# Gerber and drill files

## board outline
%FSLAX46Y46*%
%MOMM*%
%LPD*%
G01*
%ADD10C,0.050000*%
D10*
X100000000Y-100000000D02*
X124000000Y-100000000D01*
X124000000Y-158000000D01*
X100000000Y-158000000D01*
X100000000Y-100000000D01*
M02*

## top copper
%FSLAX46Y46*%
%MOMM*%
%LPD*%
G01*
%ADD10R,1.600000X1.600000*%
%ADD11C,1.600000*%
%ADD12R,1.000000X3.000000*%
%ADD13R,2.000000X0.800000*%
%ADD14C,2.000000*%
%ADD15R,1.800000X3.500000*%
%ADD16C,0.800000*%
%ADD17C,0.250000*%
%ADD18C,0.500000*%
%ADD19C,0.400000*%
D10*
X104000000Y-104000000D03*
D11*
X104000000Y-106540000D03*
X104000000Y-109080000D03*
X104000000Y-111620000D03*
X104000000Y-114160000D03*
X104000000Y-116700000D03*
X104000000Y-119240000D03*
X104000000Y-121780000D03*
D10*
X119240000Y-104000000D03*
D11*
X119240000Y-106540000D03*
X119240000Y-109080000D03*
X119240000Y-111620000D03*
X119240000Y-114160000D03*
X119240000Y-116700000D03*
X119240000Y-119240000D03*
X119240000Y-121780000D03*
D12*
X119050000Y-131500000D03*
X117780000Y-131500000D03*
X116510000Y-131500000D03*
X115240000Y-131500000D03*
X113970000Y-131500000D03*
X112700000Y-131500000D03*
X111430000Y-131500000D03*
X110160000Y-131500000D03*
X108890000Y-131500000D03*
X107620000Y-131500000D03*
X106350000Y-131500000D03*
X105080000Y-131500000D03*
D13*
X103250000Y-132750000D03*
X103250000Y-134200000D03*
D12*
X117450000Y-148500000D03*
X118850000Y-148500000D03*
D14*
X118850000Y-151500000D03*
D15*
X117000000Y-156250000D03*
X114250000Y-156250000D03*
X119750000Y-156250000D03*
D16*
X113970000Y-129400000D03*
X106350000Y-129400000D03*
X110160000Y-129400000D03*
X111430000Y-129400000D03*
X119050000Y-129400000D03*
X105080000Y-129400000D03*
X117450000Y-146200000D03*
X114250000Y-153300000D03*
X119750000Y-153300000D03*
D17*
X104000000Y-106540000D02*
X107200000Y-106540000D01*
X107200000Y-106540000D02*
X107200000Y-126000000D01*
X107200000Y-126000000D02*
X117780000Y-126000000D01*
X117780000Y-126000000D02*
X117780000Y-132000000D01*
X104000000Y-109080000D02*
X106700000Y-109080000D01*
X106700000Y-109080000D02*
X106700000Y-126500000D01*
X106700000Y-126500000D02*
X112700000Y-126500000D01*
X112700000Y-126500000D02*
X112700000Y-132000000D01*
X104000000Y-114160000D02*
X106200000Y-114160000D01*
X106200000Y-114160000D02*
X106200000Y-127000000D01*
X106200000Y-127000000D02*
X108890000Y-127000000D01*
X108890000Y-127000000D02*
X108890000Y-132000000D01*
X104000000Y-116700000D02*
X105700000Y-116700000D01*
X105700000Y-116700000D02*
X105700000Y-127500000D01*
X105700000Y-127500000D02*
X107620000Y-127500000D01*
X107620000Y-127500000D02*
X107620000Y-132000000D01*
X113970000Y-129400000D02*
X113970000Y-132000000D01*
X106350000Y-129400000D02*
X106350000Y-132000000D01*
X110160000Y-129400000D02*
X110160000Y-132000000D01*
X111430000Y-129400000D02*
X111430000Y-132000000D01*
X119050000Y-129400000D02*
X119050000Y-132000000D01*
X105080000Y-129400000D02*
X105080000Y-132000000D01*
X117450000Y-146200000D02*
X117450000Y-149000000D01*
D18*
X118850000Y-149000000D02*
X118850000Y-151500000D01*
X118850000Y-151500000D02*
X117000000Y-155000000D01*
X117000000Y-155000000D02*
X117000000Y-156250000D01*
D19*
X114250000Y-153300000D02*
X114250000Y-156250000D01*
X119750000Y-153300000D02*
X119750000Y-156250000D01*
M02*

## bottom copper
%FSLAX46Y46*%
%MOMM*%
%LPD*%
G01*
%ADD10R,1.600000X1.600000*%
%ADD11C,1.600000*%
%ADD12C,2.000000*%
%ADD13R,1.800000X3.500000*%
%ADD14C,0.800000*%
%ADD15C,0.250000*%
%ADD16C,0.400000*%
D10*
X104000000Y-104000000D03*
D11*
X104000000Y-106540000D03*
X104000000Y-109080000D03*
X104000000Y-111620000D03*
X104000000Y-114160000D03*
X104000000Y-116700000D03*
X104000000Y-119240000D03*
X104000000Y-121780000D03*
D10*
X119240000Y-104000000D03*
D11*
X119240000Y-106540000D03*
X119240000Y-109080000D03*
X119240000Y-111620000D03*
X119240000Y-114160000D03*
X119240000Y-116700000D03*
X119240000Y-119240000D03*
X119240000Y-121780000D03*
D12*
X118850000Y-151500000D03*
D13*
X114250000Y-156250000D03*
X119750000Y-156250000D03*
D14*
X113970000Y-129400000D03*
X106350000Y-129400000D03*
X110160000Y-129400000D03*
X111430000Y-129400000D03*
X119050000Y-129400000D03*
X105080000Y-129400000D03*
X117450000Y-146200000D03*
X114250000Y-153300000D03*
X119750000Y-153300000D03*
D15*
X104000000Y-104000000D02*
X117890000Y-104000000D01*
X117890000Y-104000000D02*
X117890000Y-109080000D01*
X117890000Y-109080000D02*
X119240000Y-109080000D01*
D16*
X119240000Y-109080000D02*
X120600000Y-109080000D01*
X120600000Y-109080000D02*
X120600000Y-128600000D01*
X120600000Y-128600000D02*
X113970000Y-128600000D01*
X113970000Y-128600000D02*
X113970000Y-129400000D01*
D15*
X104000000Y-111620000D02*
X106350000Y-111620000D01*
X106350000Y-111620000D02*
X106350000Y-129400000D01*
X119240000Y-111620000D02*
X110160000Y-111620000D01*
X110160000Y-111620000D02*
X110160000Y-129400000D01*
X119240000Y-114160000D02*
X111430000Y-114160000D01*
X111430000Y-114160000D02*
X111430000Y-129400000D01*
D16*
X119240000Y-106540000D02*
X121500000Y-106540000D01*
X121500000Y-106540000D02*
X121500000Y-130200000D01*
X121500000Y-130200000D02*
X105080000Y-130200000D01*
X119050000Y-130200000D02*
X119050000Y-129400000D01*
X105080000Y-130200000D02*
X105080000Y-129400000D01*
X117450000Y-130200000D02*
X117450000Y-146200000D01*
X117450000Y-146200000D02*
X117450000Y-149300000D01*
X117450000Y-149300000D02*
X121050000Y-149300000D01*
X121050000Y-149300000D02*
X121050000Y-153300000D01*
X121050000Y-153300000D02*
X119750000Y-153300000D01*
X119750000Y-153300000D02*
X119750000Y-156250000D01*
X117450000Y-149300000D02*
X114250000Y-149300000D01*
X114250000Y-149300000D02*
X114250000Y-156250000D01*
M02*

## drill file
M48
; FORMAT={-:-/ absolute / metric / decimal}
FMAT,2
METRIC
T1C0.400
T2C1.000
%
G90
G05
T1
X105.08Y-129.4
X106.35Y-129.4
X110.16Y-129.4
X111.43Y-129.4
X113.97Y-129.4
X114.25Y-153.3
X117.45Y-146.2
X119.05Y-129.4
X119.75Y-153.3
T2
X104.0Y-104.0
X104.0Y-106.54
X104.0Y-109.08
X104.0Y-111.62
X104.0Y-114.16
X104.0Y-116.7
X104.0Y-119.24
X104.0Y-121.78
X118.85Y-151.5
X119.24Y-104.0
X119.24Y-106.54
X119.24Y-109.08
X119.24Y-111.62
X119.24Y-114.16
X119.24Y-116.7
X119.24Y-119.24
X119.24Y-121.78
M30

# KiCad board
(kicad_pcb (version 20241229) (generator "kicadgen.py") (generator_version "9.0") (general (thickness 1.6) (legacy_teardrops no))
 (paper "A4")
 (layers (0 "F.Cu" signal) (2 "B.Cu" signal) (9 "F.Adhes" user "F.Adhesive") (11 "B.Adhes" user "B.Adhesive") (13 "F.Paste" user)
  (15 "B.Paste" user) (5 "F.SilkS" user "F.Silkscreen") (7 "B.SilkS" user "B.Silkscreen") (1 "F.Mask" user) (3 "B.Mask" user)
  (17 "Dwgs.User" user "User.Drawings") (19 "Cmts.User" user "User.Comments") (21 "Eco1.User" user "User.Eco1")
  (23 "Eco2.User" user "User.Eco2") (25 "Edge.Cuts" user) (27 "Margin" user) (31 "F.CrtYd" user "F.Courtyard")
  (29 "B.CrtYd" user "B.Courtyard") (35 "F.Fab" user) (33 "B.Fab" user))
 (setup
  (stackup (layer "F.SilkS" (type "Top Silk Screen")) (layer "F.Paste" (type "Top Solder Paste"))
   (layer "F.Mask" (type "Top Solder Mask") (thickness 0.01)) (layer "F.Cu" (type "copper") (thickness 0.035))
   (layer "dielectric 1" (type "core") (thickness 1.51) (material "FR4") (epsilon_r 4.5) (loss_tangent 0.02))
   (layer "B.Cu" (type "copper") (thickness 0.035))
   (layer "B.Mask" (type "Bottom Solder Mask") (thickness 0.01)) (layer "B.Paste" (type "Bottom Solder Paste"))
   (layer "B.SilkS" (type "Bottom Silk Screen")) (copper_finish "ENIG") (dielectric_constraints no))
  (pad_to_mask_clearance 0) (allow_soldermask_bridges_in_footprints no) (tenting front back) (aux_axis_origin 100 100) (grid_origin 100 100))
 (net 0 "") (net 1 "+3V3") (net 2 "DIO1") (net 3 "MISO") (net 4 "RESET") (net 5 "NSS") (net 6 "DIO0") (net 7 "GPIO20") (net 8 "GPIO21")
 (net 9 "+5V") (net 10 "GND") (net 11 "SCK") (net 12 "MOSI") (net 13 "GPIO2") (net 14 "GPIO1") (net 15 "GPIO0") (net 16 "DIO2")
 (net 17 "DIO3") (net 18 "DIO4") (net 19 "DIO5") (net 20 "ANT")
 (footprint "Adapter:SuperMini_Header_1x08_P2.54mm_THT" (layer "F.Cu") (at 104 104)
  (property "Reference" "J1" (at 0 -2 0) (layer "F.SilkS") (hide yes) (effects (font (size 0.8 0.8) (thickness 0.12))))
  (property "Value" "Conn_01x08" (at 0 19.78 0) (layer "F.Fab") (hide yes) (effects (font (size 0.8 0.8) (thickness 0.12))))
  (pad "1" thru_hole rect (at 0 0) (size 1.6 1.6) (drill 1) (layers "*.Cu" "*.Mask") (remove_unused_layers no) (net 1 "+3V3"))
  (pad "2" thru_hole circle (at 0 2.54) (size 1.6 1.6) (drill 1) (layers "*.Cu" "*.Mask") (remove_unused_layers no) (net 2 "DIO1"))
  (pad "3" thru_hole circle (at 0 5.08) (size 1.6 1.6) (drill 1) (layers "*.Cu" "*.Mask") (remove_unused_layers no) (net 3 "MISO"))
  (pad "4" thru_hole circle (at 0 7.62) (size 1.6 1.6) (drill 1) (layers "*.Cu" "*.Mask") (remove_unused_layers no) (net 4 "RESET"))
  (pad "5" thru_hole circle (at 0 10.16) (size 1.6 1.6) (drill 1) (layers "*.Cu" "*.Mask") (remove_unused_layers no) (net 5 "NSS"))
  (pad "6" thru_hole circle (at 0 12.7) (size 1.6 1.6) (drill 1) (layers "*.Cu" "*.Mask") (remove_unused_layers no) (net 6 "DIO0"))
  (pad "7" thru_hole circle (at 0 15.24) (size 1.6 1.6) (drill 1) (layers "*.Cu" "*.Mask") (remove_unused_layers no) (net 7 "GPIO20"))
  (pad "8" thru_hole circle (at 0 17.78) (size 1.6 1.6) (drill 1) (layers "*.Cu" "*.Mask") (remove_unused_layers no) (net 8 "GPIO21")))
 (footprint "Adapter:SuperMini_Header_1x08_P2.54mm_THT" (layer "F.Cu") (at 119.24 104)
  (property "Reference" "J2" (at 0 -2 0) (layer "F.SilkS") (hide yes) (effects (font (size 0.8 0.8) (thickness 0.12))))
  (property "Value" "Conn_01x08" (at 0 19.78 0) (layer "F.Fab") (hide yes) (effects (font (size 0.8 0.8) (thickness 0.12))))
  (pad "1" thru_hole rect (at 0 0) (size 1.6 1.6) (drill 1) (layers "*.Cu" "*.Mask") (remove_unused_layers no) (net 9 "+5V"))
  (pad "2" thru_hole circle (at 0 2.54) (size 1.6 1.6) (drill 1) (layers "*.Cu" "*.Mask") (remove_unused_layers no) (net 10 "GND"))
  (pad "3" thru_hole circle (at 0 5.08) (size 1.6 1.6) (drill 1) (layers "*.Cu" "*.Mask") (remove_unused_layers no) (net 1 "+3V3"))
  (pad "4" thru_hole circle (at 0 7.62) (size 1.6 1.6) (drill 1) (layers "*.Cu" "*.Mask") (remove_unused_layers no) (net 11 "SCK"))
  (pad "5" thru_hole circle (at 0 10.16) (size 1.6 1.6) (drill 1) (layers "*.Cu" "*.Mask") (remove_unused_layers no) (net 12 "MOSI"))
  (pad "6" thru_hole circle (at 0 12.7) (size 1.6 1.6) (drill 1) (layers "*.Cu" "*.Mask") (remove_unused_layers no) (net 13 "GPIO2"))
  (pad "7" thru_hole circle (at 0 15.24) (size 1.6 1.6) (drill 1) (layers "*.Cu" "*.Mask") (remove_unused_layers no) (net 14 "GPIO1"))
  (pad "8" thru_hole circle (at 0 17.78) (size 1.6 1.6) (drill 1) (layers "*.Cu" "*.Mask") (remove_unused_layers no) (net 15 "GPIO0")))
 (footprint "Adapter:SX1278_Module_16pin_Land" (layer "F.Cu") (at 103.75 131.5)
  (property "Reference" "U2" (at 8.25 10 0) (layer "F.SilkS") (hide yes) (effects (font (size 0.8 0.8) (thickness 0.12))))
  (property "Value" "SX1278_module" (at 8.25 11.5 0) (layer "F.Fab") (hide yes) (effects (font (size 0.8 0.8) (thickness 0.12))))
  (pad "1" smd rect (at 15.3 0) (size 1 3) (layers "F.Cu" "F.Mask" "F.Paste") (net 10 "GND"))
  (pad "2" smd rect (at 14.03 0) (size 1 3) (layers "F.Cu" "F.Mask" "F.Paste") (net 2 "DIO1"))
  (pad "3" smd rect (at 12.76 0) (size 1 3) (layers "F.Cu" "F.Mask" "F.Paste") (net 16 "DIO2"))
  (pad "4" smd rect (at 11.49 0) (size 1 3) (layers "F.Cu" "F.Mask" "F.Paste") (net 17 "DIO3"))
  (pad "5" smd rect (at 10.22 0) (size 1 3) (layers "F.Cu" "F.Mask" "F.Paste") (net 1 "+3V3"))
  (pad "6" smd rect (at 8.95 0) (size 1 3) (layers "F.Cu" "F.Mask" "F.Paste") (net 3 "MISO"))
  (pad "7" smd rect (at 7.68 0) (size 1 3) (layers "F.Cu" "F.Mask" "F.Paste") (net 12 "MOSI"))
  (pad "8" smd rect (at 6.41 0) (size 1 3) (layers "F.Cu" "F.Mask" "F.Paste") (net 11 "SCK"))
  (pad "9" smd rect (at 5.14 0) (size 1 3) (layers "F.Cu" "F.Mask" "F.Paste") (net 5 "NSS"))
  (pad "10" smd rect (at 3.87 0) (size 1 3) (layers "F.Cu" "F.Mask" "F.Paste") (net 6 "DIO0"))
  (pad "11" smd rect (at 2.6 0) (size 1 3) (layers "F.Cu" "F.Mask" "F.Paste") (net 4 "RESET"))
  (pad "12" smd rect (at 1.33 0) (size 1 3) (layers "F.Cu" "F.Mask" "F.Paste") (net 10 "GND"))
  (pad "13" smd rect (at -0.5 1.25) (size 2 0.8) (layers "F.Cu" "F.Mask" "F.Paste") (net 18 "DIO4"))
  (pad "14" smd rect (at -0.5 2.7) (size 2 0.8) (layers "F.Cu" "F.Mask" "F.Paste") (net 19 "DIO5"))
  (pad "15" smd rect (at 13.7 17) (size 1 3) (layers "F.Cu" "F.Mask" "F.Paste") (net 10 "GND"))
  (pad "16" smd rect (at 15.1 17) (size 1 3) (layers "F.Cu" "F.Mask" "F.Paste") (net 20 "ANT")))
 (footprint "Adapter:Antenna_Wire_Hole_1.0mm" (layer "F.Cu") (at 118.85 151.5)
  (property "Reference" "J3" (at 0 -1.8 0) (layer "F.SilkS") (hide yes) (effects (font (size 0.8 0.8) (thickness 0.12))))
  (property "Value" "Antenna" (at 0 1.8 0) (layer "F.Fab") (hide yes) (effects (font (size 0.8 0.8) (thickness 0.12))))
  (pad "1" thru_hole circle (at 0 0) (size 2 2) (drill 1) (layers "*.Cu" "*.Mask") (remove_unused_layers no) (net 20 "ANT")))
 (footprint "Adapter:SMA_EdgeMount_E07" (layer "F.Cu") (at 117 158)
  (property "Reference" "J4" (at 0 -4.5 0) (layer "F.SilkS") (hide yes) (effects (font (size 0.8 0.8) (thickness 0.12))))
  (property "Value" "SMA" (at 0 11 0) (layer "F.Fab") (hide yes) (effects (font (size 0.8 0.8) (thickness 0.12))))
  (pad "1" smd rect (at 0 -1.75) (size 1.8 3.5) (layers "F.Cu" "F.Mask" "F.Paste") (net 20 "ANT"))
  (pad "2" smd rect (at -2.75 -1.75) (size 1.8 3.5) (layers "F.Cu" "F.Mask" "F.Paste") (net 10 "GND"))
  (pad "2" smd rect (at -2.75 -1.75) (size 1.8 3.5) (layers "B.Cu" "B.Mask" "B.Paste") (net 10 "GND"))
  (pad "2" smd rect (at 2.75 -1.75) (size 1.8 3.5) (layers "F.Cu" "F.Mask" "F.Paste") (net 10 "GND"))
  (pad "2" smd rect (at 2.75 -1.75) (size 1.8 3.5) (layers "B.Cu" "B.Mask" "B.Paste") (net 10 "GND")))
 (gr_rect (start 100 100) (end 124 158) (stroke (width 0.05) (type solid)) (fill no) (layer "Edge.Cuts"))
 (segment (start 104 106.54) (end 107.2 106.54) (width 0.25) (layer "F.Cu") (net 2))
 (segment (start 107.2 106.54) (end 107.2 126) (width 0.25) (layer "F.Cu") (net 2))
 (segment (start 107.2 126) (end 117.78 126) (width 0.25) (layer "F.Cu") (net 2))
 (segment (start 117.78 126) (end 117.78 132) (width 0.25) (layer "F.Cu") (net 2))
 (segment (start 104 109.08) (end 106.7 109.08) (width 0.25) (layer "F.Cu") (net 3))
 (segment (start 106.7 109.08) (end 106.7 126.5) (width 0.25) (layer "F.Cu") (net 3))
 (segment (start 106.7 126.5) (end 112.7 126.5) (width 0.25) (layer "F.Cu") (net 3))
 (segment (start 112.7 126.5) (end 112.7 132) (width 0.25) (layer "F.Cu") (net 3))
 (segment (start 104 114.16) (end 106.2 114.16) (width 0.25) (layer "F.Cu") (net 5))
 (segment (start 106.2 114.16) (end 106.2 127) (width 0.25) (layer "F.Cu") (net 5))
 (segment (start 106.2 127) (end 108.89 127) (width 0.25) (layer "F.Cu") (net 5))
 (segment (start 108.89 127) (end 108.89 132) (width 0.25) (layer "F.Cu") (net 5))
 (segment (start 104 116.7) (end 105.7 116.7) (width 0.25) (layer "F.Cu") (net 6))
 (segment (start 105.7 116.7) (end 105.7 127.5) (width 0.25) (layer "F.Cu") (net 6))
 (segment (start 105.7 127.5) (end 107.62 127.5) (width 0.25) (layer "F.Cu") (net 6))
 (segment (start 107.62 127.5) (end 107.62 132) (width 0.25) (layer "F.Cu") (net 6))
 (segment (start 104 104) (end 117.89 104) (width 0.25) (layer "B.Cu") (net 1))
 (segment (start 117.89 104) (end 117.89 109.08) (width 0.25) (layer "B.Cu") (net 1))
 (segment (start 117.89 109.08) (end 119.24 109.08) (width 0.25) (layer "B.Cu") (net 1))
 (segment (start 119.24 109.08) (end 120.6 109.08) (width 0.4) (layer "B.Cu") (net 1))
 (segment (start 120.6 109.08) (end 120.6 128.6) (width 0.4) (layer "B.Cu") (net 1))
 (segment (start 120.6 128.6) (end 113.97 128.6) (width 0.4) (layer "B.Cu") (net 1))
 (segment (start 113.97 128.6) (end 113.97 129.4) (width 0.4) (layer "B.Cu") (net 1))
 (segment (start 113.97 129.4) (end 113.97 132) (width 0.25) (layer "F.Cu") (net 1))
 (segment (start 104 111.62) (end 106.35 111.62) (width 0.25) (layer "B.Cu") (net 4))
 (segment (start 106.35 111.62) (end 106.35 129.4) (width 0.25) (layer "B.Cu") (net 4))
 (segment (start 106.35 129.4) (end 106.35 132) (width 0.25) (layer "F.Cu") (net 4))
 (segment (start 119.24 111.62) (end 110.16 111.62) (width 0.25) (layer "B.Cu") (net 11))
 (segment (start 110.16 111.62) (end 110.16 129.4) (width 0.25) (layer "B.Cu") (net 11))
 (segment (start 110.16 129.4) (end 110.16 132) (width 0.25) (layer "F.Cu") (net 11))
 (segment (start 119.24 114.16) (end 111.43 114.16) (width 0.25) (layer "B.Cu") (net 12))
 (segment (start 111.43 114.16) (end 111.43 129.4) (width 0.25) (layer "B.Cu") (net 12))
 (segment (start 111.43 129.4) (end 111.43 132) (width 0.25) (layer "F.Cu") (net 12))
 (segment (start 119.24 106.54) (end 121.5 106.54) (width 0.4) (layer "B.Cu") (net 10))
 (segment (start 121.5 106.54) (end 121.5 130.2) (width 0.4) (layer "B.Cu") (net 10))
 (segment (start 121.5 130.2) (end 105.08 130.2) (width 0.4) (layer "B.Cu") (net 10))
 (segment (start 119.05 130.2) (end 119.05 129.4) (width 0.4) (layer "B.Cu") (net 10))
 (segment (start 119.05 129.4) (end 119.05 132) (width 0.25) (layer "F.Cu") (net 10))
 (segment (start 105.08 130.2) (end 105.08 129.4) (width 0.4) (layer "B.Cu") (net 10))
 (segment (start 105.08 129.4) (end 105.08 132) (width 0.25) (layer "F.Cu") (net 10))
 (segment (start 117.45 130.2) (end 117.45 146.2) (width 0.4) (layer "B.Cu") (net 10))
 (segment (start 117.45 146.2) (end 117.45 149) (width 0.25) (layer "F.Cu") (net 10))
 (segment (start 118.85 149) (end 118.85 151.5) (width 0.5) (layer "F.Cu") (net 20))
 (segment (start 118.85 151.5) (end 117 155) (width 0.5) (layer "F.Cu") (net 20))
 (segment (start 117 155) (end 117 156.25) (width 0.5) (layer "F.Cu") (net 20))
 (segment (start 117.45 146.2) (end 117.45 149.3) (width 0.4) (layer "B.Cu") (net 10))
 (segment (start 117.45 149.3) (end 121.05 149.3) (width 0.4) (layer "B.Cu") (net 10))
 (segment (start 121.05 149.3) (end 121.05 153.3) (width 0.4) (layer "B.Cu") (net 10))
 (segment (start 121.05 153.3) (end 119.75 153.3) (width 0.4) (layer "B.Cu") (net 10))
 (segment (start 119.75 153.3) (end 119.75 156.25) (width 0.4) (layer "B.Cu") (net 10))
 (segment (start 117.45 149.3) (end 114.25 149.3) (width 0.4) (layer "B.Cu") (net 10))
 (segment (start 114.25 149.3) (end 114.25 156.25) (width 0.4) (layer "B.Cu") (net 10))
 (segment (start 114.25 153.3) (end 114.25 156.25) (width 0.4) (layer "F.Cu") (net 10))
 (segment (start 119.75 153.3) (end 119.75 156.25) (width 0.4) (layer "F.Cu") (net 10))
 (via (at 113.97 129.4) (size 0.8) (drill 0.4) (layers "F.Cu" "B.Cu") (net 1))
 (via (at 106.35 129.4) (size 0.8) (drill 0.4) (layers "F.Cu" "B.Cu") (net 4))
 (via (at 110.16 129.4) (size 0.8) (drill 0.4) (layers "F.Cu" "B.Cu") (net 11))
 (via (at 111.43 129.4) (size 0.8) (drill 0.4) (layers "F.Cu" "B.Cu") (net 12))
 (via (at 119.05 129.4) (size 0.8) (drill 0.4) (layers "F.Cu" "B.Cu") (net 10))
 (via (at 105.08 129.4) (size 0.8) (drill 0.4) (layers "F.Cu" "B.Cu") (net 10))
 (via (at 117.45 146.2) (size 0.8) (drill 0.4) (layers "F.Cu" "B.Cu") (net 10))
 (via (at 114.25 153.3) (size 0.8) (drill 0.4) (layers "F.Cu" "B.Cu") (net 10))
 (via (at 119.75 153.3) (size 0.8) (drill 0.4) (layers "F.Cu" "B.Cu") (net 10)))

